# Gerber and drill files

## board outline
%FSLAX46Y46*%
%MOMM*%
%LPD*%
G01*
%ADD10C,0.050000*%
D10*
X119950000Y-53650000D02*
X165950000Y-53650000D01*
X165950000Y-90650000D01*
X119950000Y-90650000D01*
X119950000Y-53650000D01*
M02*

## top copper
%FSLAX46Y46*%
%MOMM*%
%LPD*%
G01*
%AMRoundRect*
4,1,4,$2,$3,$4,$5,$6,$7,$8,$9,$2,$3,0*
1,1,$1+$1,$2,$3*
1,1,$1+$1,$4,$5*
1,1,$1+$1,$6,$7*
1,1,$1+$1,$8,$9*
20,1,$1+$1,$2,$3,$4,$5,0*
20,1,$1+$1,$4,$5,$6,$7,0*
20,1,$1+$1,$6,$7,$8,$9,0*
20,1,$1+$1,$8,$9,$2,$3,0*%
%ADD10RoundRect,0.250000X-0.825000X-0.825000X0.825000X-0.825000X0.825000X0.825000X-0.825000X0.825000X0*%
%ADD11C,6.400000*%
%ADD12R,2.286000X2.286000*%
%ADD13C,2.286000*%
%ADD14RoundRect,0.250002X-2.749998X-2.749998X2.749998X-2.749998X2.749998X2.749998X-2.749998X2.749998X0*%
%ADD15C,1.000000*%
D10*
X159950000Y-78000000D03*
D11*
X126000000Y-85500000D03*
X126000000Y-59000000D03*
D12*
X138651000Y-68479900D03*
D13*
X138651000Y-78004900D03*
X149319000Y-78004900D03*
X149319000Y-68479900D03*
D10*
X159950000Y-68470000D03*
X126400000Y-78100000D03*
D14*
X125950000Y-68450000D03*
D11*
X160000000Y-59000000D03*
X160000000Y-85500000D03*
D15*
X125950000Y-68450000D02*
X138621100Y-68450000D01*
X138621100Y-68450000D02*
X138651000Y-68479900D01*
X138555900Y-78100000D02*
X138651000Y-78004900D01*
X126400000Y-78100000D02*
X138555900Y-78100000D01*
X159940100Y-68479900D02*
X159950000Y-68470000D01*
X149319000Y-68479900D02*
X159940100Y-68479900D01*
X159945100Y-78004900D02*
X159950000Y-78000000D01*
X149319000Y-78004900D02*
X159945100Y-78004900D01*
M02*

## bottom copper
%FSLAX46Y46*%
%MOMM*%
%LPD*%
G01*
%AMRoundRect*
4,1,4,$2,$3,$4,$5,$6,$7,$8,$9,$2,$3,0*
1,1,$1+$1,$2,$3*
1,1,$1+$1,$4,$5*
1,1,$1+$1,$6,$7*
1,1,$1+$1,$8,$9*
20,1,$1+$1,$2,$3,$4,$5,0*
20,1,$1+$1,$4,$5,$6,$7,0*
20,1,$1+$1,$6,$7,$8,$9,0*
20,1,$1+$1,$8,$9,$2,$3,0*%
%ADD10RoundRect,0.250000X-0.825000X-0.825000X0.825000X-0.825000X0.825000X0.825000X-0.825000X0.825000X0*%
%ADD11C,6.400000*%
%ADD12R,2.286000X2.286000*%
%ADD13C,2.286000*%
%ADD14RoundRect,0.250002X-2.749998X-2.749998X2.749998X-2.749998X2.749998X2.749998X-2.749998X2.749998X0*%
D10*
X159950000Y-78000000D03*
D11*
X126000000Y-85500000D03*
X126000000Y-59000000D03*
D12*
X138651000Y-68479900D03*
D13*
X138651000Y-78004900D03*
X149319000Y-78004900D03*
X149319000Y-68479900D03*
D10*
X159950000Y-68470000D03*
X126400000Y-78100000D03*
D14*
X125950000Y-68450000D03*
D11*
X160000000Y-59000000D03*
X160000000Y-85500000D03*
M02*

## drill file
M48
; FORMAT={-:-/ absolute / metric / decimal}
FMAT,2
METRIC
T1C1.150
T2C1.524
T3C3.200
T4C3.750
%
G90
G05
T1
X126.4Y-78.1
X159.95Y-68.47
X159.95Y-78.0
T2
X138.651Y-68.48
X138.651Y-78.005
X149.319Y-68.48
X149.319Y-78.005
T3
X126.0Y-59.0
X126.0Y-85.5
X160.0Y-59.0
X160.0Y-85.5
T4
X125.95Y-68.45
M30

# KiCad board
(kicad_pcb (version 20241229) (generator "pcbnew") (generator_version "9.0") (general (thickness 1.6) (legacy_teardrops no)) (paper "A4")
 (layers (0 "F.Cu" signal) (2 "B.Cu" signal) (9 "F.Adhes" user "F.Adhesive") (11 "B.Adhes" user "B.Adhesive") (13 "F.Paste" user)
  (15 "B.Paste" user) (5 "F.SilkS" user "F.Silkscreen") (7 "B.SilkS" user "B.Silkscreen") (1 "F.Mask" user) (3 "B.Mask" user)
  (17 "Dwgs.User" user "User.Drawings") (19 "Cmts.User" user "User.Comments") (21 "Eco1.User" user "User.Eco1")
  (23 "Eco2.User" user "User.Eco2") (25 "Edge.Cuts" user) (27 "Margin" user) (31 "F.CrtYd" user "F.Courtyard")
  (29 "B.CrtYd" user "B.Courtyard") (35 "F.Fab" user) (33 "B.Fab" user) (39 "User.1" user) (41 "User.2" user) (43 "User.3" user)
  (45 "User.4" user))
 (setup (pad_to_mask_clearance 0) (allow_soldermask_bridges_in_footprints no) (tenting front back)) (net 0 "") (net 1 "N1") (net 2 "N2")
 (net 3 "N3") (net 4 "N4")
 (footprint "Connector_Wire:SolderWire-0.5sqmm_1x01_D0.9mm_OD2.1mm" (layer "F.Cu") (at 159.95 78)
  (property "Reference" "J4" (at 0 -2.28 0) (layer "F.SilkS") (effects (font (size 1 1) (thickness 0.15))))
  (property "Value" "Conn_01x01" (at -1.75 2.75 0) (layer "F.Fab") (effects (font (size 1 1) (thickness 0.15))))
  (pad "1" thru_hole roundrect (at 0 0) (size 2.15 2.15) (drill 1.15) (layers "*.Cu" "*.Mask") (remove_unused_layers no)
   (roundrect_rratio 0.116279) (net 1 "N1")))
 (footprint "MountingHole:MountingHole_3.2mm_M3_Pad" (layer "F.Cu") (at 126 85.5)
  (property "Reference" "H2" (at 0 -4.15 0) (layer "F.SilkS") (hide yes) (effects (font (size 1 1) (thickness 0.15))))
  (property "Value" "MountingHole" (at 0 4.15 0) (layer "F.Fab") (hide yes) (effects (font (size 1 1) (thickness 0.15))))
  (pad "1" thru_hole circle (at 0 0) (size 6.4 6.4) (drill 3.2) (layers "*.Cu" "*.Mask") (remove_unused_layers no) (zone_connect 2)))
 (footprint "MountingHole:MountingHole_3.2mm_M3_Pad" (layer "F.Cu") (at 126 59)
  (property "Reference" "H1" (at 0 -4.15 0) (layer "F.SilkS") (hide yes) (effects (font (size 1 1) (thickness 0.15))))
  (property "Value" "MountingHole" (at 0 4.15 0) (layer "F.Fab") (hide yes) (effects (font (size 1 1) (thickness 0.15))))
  (pad "1" thru_hole circle (at 0 0) (size 6.4 6.4) (drill 3.2) (layers "*.Cu" "*.Mask") (remove_unused_layers no) (zone_connect 2)))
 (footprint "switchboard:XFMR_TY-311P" (layer "F.Cu") (at 143.985 73.2424)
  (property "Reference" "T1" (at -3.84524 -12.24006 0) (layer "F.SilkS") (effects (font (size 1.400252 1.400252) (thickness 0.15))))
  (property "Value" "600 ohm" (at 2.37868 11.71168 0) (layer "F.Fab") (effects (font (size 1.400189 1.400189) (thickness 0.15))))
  (pad "1" thru_hole rect (at -5.334 -4.7625) (size 2.286 2.286) (drill 1.524) (layers "*.Cu" "*.Mask") (remove_unused_layers no)
   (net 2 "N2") (solder_mask_margin 0.102))
  (pad "3" thru_hole circle (at -5.334 4.7625) (size 2.286 2.286) (drill 1.524) (layers "*.Cu" "*.Mask") (remove_unused_layers no)
   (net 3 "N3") (solder_mask_margin 0.102))
  (pad "4" thru_hole circle (at 5.334 4.7625) (size 2.286 2.286) (drill 1.524) (layers "*.Cu" "*.Mask") (remove_unused_layers no)
   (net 1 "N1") (solder_mask_margin 0.102))
  (pad "6" thru_hole circle (at 5.334 -4.7625) (size 2.286 2.286) (drill 1.524) (layers "*.Cu" "*.Mask") (remove_unused_layers no)
   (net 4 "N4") (solder_mask_margin 0.102)))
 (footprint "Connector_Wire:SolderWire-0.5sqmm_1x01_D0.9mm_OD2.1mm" (layer "F.Cu") (at 159.95 68.47)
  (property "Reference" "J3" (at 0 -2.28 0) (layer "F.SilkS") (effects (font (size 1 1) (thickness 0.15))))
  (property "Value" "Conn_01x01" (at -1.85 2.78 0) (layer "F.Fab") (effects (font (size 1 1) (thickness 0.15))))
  (pad "1" thru_hole roundrect (at 0 0) (size 2.15 2.15) (drill 1.15) (layers "*.Cu" "*.Mask") (remove_unused_layers no)
   (roundrect_rratio 0.116279) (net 4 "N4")))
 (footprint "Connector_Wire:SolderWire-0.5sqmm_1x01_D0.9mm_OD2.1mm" (layer "F.Cu") (at 126.4 78.1)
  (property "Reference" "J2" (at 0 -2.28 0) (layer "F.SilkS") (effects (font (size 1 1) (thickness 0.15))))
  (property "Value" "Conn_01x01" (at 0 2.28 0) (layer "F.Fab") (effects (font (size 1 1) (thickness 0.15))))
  (pad "1" thru_hole roundrect (at 0 0) (size 2.15 2.15) (drill 1.15) (layers "*.Cu" "*.Mask") (remove_unused_layers no)
   (roundrect_rratio 0.116279) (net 3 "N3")))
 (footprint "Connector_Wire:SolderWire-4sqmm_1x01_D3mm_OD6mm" (layer "F.Cu") (at 125.95 68.45)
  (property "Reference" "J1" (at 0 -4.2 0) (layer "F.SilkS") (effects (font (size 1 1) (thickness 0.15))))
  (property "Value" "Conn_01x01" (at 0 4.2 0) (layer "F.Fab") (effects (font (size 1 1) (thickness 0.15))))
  (pad "1" thru_hole roundrect (at 0 0) (size 6 6) (drill 3.75) (layers "*.Cu" "*.Mask") (remove_unused_layers no)
   (roundrect_rratio 0.041667) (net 2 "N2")))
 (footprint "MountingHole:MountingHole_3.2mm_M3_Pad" (layer "F.Cu") (at 160 59)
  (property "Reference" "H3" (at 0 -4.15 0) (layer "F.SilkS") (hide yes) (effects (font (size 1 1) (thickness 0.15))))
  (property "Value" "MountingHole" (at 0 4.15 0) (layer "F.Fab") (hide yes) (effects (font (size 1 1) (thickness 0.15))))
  (pad "1" thru_hole circle (at 0 0) (size 6.4 6.4) (drill 3.2) (layers "*.Cu" "*.Mask") (remove_unused_layers no) (zone_connect 2)))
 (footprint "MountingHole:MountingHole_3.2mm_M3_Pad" (layer "F.Cu") (at 160 85.5)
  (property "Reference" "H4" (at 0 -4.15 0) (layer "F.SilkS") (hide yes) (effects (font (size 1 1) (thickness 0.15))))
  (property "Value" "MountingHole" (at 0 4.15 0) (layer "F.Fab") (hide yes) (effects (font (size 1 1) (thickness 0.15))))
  (pad "1" thru_hole circle (at 0 0) (size 6.4 6.4) (drill 3.2) (layers "*.Cu" "*.Mask") (remove_unused_layers no) (zone_connect 2)))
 (gr_rect (start 119.95 53.65) (end 165.95 90.65) (stroke (width 0.05) (type solid)) (fill no) (layer "Edge.Cuts"))
 (segment (start 125.95 68.45) (end 138.6211 68.45) (width 1) (layer "F.Cu") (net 2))
 (segment (start 138.6211 68.45) (end 138.651 68.4799) (width 1) (layer "F.Cu") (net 2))
 (segment (start 138.5559 78.1) (end 138.651 78.0049) (width 1) (layer "F.Cu") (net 3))
 (segment (start 126.4 78.1) (end 138.5559 78.1) (width 1) (layer "F.Cu") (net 3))
 (segment (start 159.9401 68.4799) (end 159.95 68.47) (width 1) (layer "F.Cu") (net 4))
 (segment (start 149.319 68.4799) (end 159.9401 68.4799) (width 1) (layer "F.Cu") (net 4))
 (segment (start 159.9451 78.0049) (end 159.95 78) (width 1) (layer "F.Cu") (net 1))
 (segment (start 149.319 78.0049) (end 159.9451 78.0049) (width 1) (layer "F.Cu") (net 1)))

